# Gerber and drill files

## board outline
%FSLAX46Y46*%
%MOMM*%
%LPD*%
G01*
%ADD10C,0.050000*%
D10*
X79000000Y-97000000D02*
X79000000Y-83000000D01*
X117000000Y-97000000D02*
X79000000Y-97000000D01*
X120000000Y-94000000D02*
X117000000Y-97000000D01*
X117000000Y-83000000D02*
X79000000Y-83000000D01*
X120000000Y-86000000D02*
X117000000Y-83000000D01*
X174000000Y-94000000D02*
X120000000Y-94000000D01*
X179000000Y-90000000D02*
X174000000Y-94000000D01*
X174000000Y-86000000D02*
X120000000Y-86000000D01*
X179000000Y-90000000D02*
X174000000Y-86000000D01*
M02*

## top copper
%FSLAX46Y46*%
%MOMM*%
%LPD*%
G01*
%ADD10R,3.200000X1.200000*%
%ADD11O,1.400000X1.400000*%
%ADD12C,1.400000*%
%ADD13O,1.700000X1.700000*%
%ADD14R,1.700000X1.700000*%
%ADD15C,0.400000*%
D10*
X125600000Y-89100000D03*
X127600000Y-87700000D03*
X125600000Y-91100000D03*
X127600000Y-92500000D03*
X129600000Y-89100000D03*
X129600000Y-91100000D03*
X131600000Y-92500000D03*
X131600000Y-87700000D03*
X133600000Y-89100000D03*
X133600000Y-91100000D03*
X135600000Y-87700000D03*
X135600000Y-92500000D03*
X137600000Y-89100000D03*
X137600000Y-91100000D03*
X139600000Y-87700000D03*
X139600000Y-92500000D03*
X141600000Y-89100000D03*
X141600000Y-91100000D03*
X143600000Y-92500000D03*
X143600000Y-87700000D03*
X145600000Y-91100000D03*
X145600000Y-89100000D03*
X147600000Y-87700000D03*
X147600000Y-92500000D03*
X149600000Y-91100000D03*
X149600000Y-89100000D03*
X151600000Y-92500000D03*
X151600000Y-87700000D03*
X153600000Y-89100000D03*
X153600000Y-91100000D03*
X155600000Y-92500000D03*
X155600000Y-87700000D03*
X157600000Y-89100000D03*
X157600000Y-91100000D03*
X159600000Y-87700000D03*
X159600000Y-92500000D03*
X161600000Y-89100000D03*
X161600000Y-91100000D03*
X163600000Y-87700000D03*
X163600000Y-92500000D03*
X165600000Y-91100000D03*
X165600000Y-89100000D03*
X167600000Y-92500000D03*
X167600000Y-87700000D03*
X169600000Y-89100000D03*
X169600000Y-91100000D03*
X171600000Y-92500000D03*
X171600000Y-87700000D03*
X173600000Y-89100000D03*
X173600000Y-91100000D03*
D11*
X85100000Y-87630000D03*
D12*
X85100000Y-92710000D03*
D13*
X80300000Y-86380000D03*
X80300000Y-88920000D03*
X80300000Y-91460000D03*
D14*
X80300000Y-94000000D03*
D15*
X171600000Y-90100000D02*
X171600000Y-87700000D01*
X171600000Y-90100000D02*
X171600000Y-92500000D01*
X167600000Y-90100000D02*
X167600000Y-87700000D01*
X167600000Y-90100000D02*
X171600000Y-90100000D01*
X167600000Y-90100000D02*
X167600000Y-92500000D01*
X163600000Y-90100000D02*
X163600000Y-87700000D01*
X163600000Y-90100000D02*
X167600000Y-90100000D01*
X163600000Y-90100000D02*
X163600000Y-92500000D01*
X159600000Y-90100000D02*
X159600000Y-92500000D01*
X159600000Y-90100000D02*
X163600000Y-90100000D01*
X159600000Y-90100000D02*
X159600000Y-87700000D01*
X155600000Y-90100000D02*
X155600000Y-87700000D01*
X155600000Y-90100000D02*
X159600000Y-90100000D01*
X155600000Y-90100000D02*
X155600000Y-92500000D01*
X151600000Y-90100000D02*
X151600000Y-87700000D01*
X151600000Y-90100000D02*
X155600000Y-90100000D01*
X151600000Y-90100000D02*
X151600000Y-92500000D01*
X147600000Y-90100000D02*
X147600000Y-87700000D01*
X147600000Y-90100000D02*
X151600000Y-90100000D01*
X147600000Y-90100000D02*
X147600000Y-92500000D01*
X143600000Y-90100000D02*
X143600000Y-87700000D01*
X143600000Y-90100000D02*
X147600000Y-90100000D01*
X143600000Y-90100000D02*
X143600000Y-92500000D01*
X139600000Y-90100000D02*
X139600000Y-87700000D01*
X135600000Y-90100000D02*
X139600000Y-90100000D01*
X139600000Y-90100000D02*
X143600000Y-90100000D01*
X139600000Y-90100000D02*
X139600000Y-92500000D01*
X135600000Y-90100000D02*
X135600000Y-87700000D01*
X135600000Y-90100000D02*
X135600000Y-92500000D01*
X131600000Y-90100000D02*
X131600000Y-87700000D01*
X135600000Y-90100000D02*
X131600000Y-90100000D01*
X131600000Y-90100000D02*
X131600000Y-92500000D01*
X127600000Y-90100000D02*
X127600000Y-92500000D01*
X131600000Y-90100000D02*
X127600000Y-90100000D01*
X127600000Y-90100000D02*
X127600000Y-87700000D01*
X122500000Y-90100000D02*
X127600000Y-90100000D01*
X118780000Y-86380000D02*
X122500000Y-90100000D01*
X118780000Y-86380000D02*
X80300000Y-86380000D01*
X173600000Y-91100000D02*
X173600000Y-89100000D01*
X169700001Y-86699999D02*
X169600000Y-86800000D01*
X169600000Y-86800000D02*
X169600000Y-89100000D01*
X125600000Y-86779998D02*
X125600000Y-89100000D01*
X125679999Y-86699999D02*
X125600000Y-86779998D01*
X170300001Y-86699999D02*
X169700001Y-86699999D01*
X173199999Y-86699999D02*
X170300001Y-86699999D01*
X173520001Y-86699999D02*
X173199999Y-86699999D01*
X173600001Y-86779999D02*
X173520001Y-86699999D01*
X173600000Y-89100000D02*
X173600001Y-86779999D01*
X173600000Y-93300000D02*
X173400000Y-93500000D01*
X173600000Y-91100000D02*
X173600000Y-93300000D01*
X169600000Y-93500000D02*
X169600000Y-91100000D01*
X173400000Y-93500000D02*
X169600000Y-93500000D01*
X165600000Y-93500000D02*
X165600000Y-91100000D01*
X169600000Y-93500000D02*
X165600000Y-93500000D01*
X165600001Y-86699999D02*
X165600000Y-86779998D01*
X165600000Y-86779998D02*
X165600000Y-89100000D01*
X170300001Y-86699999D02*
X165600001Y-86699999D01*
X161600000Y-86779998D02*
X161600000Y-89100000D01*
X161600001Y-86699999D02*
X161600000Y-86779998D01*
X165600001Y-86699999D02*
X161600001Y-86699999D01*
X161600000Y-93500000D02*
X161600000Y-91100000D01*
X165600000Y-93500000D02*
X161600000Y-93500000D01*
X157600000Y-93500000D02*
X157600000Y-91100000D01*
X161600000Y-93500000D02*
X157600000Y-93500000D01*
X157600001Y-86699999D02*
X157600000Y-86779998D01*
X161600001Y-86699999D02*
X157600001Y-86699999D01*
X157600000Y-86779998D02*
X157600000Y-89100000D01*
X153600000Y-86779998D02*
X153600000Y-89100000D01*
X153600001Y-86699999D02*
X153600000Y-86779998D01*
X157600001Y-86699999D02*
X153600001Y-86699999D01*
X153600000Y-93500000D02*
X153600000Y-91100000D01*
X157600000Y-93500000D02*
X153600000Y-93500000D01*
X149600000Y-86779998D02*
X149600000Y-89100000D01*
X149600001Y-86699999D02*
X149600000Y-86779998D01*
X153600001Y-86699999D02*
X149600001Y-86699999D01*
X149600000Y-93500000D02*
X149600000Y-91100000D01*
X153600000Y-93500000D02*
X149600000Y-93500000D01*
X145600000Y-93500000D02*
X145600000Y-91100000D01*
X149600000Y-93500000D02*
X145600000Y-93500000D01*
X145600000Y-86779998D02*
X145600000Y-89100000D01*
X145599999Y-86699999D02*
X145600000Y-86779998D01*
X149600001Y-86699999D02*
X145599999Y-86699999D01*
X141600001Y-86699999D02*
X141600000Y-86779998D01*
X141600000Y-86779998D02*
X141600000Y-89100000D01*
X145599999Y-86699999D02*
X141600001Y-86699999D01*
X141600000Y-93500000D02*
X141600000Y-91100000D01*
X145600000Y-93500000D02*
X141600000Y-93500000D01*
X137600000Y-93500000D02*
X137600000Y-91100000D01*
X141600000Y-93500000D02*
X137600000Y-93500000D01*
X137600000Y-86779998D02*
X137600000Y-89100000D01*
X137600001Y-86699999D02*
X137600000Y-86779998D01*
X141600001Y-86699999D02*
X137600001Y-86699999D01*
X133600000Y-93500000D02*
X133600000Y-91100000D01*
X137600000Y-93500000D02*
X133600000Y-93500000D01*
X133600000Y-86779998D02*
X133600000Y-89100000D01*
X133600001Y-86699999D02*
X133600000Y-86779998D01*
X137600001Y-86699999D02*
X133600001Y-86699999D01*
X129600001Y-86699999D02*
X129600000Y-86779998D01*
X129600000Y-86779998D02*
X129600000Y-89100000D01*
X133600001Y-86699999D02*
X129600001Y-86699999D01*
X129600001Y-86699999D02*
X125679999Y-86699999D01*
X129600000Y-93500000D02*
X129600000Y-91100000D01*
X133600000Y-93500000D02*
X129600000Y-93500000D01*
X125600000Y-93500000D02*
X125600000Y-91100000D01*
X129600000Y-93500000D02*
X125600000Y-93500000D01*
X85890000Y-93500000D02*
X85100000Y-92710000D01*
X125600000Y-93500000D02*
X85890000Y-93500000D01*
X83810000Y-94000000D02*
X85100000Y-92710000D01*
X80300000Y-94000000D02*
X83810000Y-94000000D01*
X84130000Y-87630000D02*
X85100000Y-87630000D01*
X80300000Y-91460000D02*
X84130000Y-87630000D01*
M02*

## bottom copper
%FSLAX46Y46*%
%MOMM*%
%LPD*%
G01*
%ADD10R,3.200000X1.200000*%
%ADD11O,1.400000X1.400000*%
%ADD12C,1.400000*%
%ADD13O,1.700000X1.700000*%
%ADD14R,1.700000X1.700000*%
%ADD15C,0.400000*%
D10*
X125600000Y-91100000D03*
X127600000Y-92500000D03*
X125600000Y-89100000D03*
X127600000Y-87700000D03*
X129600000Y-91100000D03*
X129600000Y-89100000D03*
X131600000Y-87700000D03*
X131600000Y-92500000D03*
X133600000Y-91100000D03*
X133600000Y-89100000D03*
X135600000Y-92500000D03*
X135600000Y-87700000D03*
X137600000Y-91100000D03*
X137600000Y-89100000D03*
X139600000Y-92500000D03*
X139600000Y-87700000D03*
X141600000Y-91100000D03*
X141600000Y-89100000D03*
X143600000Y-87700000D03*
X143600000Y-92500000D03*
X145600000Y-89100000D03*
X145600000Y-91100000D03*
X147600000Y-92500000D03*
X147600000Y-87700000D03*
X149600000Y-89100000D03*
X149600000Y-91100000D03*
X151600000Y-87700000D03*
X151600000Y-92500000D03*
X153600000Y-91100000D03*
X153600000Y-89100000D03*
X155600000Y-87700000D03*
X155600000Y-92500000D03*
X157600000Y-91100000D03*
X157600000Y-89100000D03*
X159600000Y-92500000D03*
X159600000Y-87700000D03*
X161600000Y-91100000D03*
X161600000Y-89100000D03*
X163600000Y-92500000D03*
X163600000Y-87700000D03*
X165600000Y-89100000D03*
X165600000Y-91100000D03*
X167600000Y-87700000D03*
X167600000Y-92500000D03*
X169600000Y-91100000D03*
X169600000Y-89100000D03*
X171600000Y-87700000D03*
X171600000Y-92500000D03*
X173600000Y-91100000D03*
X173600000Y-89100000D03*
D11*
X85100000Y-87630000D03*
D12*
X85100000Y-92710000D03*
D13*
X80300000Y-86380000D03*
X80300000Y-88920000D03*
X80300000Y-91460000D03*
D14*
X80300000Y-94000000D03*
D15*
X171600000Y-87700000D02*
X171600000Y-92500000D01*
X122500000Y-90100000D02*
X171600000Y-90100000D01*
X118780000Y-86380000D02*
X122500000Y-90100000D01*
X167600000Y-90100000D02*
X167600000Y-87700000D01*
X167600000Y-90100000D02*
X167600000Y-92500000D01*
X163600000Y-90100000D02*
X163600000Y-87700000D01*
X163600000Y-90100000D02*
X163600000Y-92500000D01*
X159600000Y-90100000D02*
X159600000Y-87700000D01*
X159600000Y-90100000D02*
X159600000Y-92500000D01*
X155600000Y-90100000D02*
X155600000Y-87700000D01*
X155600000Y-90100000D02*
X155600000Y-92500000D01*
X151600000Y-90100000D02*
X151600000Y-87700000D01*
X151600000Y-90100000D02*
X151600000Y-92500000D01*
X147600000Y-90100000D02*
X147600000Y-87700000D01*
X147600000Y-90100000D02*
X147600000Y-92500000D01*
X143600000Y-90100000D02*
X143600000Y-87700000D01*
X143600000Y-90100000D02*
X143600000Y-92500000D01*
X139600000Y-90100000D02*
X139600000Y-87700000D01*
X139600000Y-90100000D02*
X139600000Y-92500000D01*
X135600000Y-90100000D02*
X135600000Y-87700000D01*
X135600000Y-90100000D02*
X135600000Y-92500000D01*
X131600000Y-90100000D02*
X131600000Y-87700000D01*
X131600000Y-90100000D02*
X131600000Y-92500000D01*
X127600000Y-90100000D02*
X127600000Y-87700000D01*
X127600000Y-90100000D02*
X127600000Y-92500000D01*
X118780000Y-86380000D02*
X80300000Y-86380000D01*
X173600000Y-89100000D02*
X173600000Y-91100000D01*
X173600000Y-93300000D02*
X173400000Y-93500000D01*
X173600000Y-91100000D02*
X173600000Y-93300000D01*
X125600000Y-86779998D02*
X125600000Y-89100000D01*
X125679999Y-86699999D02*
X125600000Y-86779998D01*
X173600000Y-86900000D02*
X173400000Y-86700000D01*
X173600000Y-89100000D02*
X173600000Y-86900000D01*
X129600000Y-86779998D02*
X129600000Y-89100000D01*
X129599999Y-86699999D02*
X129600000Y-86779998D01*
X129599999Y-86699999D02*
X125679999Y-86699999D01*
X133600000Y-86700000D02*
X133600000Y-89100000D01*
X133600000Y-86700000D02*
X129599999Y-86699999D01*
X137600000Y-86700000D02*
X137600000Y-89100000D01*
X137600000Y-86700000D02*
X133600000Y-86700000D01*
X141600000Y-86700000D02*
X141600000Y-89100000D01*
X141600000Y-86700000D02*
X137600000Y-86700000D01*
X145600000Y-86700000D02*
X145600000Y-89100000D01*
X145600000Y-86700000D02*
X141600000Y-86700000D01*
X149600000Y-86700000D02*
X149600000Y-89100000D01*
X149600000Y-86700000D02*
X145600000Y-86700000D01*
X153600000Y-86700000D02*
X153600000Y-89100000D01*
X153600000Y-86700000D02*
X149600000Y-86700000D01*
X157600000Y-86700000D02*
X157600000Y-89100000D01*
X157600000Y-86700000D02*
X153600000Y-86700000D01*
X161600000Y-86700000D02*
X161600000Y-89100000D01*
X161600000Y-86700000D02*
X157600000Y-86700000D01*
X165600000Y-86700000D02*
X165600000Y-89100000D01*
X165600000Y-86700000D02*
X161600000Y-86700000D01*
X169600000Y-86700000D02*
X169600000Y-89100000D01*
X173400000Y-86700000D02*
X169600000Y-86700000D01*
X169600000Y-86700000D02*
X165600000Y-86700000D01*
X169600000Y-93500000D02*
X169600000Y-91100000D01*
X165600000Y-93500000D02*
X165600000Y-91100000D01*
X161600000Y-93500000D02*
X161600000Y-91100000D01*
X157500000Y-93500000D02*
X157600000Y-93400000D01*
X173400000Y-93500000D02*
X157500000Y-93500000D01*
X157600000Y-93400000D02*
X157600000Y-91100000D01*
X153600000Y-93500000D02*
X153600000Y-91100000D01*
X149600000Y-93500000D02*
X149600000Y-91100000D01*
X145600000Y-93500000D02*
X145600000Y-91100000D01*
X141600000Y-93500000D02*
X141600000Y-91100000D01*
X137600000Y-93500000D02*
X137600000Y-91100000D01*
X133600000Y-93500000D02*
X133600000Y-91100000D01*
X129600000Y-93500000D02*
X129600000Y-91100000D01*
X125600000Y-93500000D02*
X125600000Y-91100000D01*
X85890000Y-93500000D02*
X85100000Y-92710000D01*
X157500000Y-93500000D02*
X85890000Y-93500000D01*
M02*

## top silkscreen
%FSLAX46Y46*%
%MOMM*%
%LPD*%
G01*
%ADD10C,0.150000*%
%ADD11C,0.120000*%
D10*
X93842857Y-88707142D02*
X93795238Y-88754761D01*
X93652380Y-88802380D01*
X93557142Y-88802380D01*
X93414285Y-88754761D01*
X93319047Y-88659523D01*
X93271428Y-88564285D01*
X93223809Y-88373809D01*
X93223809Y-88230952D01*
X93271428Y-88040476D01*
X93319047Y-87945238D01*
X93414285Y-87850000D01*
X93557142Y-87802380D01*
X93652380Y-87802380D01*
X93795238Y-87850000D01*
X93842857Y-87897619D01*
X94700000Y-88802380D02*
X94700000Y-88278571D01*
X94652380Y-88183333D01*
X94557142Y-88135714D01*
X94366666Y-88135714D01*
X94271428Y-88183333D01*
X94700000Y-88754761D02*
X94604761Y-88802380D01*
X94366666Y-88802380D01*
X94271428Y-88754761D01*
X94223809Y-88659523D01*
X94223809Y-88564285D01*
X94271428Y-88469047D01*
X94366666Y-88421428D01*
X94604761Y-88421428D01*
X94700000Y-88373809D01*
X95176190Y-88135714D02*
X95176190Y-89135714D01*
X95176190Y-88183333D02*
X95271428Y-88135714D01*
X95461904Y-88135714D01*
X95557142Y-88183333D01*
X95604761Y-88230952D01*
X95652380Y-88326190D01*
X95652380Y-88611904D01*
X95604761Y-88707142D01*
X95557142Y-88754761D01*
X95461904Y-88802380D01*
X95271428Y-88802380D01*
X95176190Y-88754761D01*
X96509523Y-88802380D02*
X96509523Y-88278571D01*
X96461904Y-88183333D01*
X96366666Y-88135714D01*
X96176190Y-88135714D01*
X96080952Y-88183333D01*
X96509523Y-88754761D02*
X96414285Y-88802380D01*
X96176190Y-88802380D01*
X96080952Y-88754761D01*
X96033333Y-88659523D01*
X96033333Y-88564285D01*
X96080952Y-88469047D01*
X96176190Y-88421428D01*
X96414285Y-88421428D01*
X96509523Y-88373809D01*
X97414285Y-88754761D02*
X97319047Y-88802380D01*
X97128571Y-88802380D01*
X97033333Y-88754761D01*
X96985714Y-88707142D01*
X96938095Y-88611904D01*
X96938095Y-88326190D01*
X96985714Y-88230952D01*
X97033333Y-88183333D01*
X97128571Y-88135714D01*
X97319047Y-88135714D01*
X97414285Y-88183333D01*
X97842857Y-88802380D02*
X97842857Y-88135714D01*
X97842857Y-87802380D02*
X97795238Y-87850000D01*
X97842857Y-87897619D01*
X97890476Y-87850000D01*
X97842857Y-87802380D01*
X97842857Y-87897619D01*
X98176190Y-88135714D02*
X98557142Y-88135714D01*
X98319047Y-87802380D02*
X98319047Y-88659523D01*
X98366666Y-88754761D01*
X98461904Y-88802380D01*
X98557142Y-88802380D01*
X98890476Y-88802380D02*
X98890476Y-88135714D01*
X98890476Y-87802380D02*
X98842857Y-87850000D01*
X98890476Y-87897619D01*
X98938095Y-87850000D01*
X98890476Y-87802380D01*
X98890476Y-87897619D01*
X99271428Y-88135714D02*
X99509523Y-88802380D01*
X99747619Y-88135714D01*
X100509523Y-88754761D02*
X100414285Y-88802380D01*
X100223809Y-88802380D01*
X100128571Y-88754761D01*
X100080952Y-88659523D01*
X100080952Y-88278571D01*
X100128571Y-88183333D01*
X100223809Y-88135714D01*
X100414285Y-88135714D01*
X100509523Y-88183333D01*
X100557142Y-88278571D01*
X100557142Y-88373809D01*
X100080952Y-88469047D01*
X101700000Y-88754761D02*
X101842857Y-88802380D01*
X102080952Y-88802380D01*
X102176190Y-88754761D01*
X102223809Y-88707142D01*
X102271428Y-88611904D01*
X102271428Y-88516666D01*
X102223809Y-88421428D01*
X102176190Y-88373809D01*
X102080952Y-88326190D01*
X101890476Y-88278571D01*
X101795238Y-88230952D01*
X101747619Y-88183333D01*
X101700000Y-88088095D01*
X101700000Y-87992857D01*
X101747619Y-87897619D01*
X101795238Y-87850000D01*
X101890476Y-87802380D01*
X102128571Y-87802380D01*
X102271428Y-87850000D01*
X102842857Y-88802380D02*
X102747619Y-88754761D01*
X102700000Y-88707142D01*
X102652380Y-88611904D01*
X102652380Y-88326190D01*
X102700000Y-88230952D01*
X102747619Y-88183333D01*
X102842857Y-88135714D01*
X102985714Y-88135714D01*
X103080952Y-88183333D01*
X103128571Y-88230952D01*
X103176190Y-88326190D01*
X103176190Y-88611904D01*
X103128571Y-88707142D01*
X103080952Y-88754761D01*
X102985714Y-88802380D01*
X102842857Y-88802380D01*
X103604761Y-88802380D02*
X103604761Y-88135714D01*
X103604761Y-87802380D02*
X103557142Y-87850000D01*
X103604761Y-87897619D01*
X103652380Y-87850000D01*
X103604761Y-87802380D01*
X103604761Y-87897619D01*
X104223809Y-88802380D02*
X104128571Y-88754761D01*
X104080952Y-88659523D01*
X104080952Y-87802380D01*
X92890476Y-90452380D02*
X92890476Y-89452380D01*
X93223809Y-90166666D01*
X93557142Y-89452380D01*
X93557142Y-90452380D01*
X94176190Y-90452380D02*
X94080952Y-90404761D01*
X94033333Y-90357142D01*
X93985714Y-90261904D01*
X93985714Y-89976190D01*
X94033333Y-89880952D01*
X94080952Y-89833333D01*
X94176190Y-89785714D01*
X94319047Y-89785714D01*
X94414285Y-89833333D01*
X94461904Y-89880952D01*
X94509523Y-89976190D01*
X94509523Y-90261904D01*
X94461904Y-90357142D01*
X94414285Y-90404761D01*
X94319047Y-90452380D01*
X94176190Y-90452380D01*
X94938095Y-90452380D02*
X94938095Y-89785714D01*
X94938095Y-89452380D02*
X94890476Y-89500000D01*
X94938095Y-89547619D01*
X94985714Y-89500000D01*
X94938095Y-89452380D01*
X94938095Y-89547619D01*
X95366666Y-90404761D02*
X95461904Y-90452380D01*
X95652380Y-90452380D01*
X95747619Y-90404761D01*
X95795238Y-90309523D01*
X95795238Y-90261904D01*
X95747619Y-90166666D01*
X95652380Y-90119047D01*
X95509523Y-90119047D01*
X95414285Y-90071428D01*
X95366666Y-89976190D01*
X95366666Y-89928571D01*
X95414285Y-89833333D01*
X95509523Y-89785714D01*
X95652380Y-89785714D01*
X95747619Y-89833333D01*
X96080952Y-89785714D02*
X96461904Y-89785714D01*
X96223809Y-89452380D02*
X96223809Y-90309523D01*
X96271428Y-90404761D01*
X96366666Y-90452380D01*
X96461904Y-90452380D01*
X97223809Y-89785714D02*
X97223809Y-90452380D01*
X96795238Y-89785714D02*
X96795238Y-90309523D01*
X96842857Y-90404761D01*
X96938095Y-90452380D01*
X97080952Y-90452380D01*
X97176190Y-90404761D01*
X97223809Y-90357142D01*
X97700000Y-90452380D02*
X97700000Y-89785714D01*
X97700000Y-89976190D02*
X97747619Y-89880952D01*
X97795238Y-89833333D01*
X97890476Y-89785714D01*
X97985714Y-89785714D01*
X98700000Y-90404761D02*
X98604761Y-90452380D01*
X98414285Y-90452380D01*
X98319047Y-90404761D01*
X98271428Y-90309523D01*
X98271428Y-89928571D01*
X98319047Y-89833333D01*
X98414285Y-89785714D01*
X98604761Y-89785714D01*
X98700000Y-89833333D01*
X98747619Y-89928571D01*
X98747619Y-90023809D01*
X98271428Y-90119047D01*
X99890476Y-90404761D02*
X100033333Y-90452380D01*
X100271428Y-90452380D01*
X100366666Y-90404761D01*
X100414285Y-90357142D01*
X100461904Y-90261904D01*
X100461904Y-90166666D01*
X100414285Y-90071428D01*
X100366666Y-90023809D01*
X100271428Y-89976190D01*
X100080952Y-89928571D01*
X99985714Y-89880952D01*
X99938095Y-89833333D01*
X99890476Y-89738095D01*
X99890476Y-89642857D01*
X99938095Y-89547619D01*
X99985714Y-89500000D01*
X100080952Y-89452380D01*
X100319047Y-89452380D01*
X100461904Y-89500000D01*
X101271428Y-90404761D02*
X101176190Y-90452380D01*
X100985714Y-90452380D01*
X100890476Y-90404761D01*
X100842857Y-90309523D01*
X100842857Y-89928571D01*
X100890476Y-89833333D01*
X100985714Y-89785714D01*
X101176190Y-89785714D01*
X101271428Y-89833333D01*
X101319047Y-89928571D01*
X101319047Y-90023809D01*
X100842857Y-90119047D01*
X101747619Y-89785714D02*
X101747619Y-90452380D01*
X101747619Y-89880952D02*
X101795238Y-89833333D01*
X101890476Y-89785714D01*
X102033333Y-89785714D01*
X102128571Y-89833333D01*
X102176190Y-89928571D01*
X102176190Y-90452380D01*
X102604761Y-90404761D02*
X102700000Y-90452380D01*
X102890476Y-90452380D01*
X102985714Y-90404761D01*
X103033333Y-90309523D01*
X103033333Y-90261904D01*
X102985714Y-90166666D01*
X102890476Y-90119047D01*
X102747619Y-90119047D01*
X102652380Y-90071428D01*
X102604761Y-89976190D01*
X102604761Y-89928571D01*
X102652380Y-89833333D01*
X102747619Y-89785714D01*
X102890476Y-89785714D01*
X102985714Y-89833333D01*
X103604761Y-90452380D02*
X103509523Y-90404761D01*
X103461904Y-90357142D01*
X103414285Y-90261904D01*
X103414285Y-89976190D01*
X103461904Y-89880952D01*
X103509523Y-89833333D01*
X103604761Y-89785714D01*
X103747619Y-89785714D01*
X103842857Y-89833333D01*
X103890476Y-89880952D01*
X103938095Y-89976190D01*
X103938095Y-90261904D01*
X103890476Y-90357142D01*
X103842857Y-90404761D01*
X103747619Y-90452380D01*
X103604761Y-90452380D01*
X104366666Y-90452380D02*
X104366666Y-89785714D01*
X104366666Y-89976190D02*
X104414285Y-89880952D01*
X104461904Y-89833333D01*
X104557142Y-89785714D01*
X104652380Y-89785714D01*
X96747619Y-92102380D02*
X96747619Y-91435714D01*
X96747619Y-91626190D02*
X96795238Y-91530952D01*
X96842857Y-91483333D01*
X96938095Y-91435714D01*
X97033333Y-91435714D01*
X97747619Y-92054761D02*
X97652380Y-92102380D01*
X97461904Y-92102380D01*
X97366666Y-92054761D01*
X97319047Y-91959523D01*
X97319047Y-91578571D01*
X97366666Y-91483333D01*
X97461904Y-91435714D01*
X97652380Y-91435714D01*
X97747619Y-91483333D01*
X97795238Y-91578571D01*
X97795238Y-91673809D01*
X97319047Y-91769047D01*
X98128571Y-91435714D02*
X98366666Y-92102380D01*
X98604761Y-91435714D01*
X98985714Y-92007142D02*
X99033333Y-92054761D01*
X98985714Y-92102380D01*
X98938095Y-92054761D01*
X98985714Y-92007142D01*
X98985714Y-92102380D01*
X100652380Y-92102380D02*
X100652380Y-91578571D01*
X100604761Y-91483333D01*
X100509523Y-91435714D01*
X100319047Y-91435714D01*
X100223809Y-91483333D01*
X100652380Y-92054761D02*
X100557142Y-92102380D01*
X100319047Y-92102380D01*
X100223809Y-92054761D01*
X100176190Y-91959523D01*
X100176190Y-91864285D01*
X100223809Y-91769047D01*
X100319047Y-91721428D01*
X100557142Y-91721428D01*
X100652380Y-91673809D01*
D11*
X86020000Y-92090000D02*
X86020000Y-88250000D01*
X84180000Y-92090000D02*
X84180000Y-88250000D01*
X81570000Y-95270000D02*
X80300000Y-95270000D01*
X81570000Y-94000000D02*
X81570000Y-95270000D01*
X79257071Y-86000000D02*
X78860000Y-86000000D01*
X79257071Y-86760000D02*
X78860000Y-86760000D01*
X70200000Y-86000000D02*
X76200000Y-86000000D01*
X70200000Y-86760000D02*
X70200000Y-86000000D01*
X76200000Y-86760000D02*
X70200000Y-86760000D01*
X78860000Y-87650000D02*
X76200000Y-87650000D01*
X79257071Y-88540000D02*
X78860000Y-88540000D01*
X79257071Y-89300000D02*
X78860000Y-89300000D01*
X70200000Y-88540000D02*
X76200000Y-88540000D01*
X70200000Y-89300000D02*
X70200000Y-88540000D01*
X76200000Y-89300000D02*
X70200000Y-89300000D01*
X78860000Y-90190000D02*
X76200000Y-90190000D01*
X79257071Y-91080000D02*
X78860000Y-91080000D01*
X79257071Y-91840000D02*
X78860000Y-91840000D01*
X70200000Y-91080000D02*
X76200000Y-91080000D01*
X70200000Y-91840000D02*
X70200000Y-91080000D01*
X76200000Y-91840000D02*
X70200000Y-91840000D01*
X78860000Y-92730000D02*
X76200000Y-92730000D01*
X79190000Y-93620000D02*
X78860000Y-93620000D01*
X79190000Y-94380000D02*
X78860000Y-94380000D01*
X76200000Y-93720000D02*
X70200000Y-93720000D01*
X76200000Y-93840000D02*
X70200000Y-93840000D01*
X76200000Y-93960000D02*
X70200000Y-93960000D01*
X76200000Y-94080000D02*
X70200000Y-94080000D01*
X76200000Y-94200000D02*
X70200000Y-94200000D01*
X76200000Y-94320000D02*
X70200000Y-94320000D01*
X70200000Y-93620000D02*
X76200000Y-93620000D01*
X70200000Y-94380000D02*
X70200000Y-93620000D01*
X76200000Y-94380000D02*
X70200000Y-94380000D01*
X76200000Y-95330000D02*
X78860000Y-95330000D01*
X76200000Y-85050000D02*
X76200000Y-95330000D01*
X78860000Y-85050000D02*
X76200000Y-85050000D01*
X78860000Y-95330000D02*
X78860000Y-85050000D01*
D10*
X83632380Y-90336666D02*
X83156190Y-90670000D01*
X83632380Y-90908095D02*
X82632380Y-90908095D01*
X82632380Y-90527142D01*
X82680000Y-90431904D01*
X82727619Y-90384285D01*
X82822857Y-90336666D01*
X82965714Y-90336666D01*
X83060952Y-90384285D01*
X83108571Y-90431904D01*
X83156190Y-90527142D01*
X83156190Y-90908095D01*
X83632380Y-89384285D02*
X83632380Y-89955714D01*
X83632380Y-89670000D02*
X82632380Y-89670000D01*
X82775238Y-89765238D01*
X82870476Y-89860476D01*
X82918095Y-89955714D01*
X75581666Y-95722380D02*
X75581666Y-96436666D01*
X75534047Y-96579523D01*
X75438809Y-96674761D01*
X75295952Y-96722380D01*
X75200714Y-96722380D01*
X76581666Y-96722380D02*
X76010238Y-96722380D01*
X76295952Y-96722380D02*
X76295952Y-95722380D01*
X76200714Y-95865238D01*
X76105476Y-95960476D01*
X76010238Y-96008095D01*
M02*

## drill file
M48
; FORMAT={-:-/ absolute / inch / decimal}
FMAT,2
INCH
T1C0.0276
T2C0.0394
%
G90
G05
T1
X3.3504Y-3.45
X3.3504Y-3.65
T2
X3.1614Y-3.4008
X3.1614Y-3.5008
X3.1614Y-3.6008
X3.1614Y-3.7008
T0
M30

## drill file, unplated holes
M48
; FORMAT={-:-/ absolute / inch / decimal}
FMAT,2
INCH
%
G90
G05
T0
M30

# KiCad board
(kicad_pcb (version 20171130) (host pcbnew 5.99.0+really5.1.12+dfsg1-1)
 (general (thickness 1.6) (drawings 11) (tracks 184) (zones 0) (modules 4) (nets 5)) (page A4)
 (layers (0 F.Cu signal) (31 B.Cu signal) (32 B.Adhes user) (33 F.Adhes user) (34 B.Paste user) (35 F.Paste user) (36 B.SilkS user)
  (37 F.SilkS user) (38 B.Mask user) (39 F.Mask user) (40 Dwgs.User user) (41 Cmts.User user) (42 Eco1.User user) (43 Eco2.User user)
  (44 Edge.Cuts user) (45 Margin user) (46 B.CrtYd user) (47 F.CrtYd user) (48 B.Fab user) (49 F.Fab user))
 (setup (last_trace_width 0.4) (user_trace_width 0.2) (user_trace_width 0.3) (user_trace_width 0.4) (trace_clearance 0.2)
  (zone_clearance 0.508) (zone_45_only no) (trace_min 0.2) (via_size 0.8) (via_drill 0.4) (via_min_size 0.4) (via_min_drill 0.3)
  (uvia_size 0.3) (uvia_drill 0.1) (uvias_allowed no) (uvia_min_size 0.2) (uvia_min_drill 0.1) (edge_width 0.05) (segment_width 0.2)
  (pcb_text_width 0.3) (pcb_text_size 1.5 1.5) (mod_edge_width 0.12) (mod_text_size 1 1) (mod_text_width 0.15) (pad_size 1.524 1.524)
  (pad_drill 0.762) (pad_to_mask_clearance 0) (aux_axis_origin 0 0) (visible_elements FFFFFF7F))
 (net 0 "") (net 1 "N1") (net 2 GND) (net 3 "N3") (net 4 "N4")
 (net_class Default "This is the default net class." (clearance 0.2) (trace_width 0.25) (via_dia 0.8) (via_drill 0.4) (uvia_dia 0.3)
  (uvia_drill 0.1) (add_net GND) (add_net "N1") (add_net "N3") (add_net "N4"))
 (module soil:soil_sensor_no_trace (layer B.Cu) (at 124 90.1)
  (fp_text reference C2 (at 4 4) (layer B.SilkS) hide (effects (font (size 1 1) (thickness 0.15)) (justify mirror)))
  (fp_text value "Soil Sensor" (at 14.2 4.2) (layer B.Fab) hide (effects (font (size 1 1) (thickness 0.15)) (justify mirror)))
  (pad 1 smd rect (at 1.6 1) (size 3.2 1.2) (layers B.Cu) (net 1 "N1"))
  (pad 2 smd rect (at 3.6 2.4) (size 3.2 1.2) (layers B.Cu) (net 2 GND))
  (pad 1 smd rect (at 1.6 -1) (size 3.2 1.2) (layers B.Cu) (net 1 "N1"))
  (pad 2 smd rect (at 3.6 -2.4) (size 3.2 1.2) (layers B.Cu) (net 2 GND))
  (pad 1 smd rect (at 5.6 1) (size 3.2 1.2) (layers B.Cu) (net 1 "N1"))
  (pad 1 smd rect (at 5.6 -1) (size 3.2 1.2) (layers B.Cu) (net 1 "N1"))
  (pad 2 smd rect (at 7.6 -2.4) (size 3.2 1.2) (layers B.Cu) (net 2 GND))
  (pad 2 smd rect (at 7.6 2.4) (size 3.2 1.2) (layers B.Cu) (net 2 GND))
  (pad 1 smd rect (at 9.6 1) (size 3.2 1.2) (layers B.Cu) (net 1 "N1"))
  (pad 1 smd rect (at 9.6 -1) (size 3.2 1.2) (layers B.Cu) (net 1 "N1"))
  (pad 2 smd rect (at 11.6 2.4) (size 3.2 1.2) (layers B.Cu) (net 2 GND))
  (pad 2 smd rect (at 11.6 -2.4) (size 3.2 1.2) (layers B.Cu) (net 2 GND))
  (pad 1 smd rect (at 13.6 1) (size 3.2 1.2) (layers B.Cu) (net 1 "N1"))
  (pad 1 smd rect (at 13.6 -1) (size 3.2 1.2) (layers B.Cu) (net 1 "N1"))
  (pad 2 smd rect (at 15.6 2.4) (size 3.2 1.2) (layers B.Cu) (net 2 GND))
  (pad 2 smd rect (at 15.6 -2.4) (size 3.2 1.2) (layers B.Cu) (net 2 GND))
  (pad 1 smd rect (at 17.6 1) (size 3.2 1.2) (layers B.Cu) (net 1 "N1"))
  (pad 1 smd rect (at 17.6 -1) (size 3.2 1.2) (layers B.Cu) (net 1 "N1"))
  (pad 2 smd rect (at 19.6 -2.4) (size 3.2 1.2) (layers B.Cu) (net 2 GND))
  (pad 2 smd rect (at 19.6 2.4) (size 3.2 1.2) (layers B.Cu) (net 2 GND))
  (pad 1 smd rect (at 21.6 -1) (size 3.2 1.2) (layers B.Cu) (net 1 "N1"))
  (pad 1 smd rect (at 21.6 1) (size 3.2 1.2) (layers B.Cu) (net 1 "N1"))
  (pad 2 smd rect (at 23.6 2.4) (size 3.2 1.2) (layers B.Cu) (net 2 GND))
  (pad 2 smd rect (at 23.6 -2.4) (size 3.2 1.2) (layers B.Cu) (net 2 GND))
  (pad 1 smd rect (at 25.6 -1) (size 3.2 1.2) (layers B.Cu) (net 1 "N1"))
  (pad 1 smd rect (at 25.6 1) (size 3.2 1.2) (layers B.Cu) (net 1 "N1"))
  (pad 2 smd rect (at 27.6 -2.4) (size 3.2 1.2) (layers B.Cu) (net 2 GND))
  (pad 2 smd rect (at 27.6 2.4) (size 3.2 1.2) (layers B.Cu) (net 2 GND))
  (pad 1 smd rect (at 29.6 1) (size 3.2 1.2) (layers B.Cu) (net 1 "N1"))
  (pad 1 smd rect (at 29.6 -1) (size 3.2 1.2) (layers B.Cu) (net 1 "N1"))
  (pad 2 smd rect (at 31.6 -2.4) (size 3.2 1.2) (layers B.Cu) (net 2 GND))
  (pad 2 smd rect (at 31.6 2.4) (size 3.2 1.2) (layers B.Cu) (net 2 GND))
  (pad 1 smd rect (at 33.6 1) (size 3.2 1.2) (layers B.Cu) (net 1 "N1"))
  (pad 1 smd rect (at 33.6 -1) (size 3.2 1.2) (layers B.Cu) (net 1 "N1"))
  (pad 2 smd rect (at 35.6 2.4) (size 3.2 1.2) (layers B.Cu) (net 2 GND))
  (pad 2 smd rect (at 35.6 -2.4) (size 3.2 1.2) (layers B.Cu) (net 2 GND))
  (pad 1 smd rect (at 37.6 1) (size 3.2 1.2) (layers B.Cu) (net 1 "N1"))
  (pad 1 smd rect (at 37.6 -1) (size 3.2 1.2) (layers B.Cu) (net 1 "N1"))
  (pad 2 smd rect (at 39.6 2.4) (size 3.2 1.2) (layers B.Cu) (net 2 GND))
  (pad 2 smd rect (at 39.6 -2.4) (size 3.2 1.2) (layers B.Cu) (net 2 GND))
  (pad 1 smd rect (at 41.6 -1) (size 3.2 1.2) (layers B.Cu) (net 1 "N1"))
  (pad 1 smd rect (at 41.6 1) (size 3.2 1.2) (layers B.Cu) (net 1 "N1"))
  (pad 2 smd rect (at 43.6 -2.4) (size 3.2 1.2) (layers B.Cu) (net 2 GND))
  (pad 2 smd rect (at 43.6 2.4) (size 3.2 1.2) (layers B.Cu) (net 2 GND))
  (pad 1 smd rect (at 45.6 1) (size 3.2 1.2) (layers B.Cu) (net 1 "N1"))
  (pad 1 smd rect (at 45.6 -1) (size 3.2 1.2) (layers B.Cu) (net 1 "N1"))
  (pad 2 smd rect (at 47.6 -2.4) (size 3.2 1.2) (layers B.Cu) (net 2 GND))
  (pad 2 smd rect (at 47.6 2.4) (size 3.2 1.2) (layers B.Cu) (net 2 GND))
  (pad 1 smd rect (at 49.6 1) (size 3.2 1.2) (layers B.Cu) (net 1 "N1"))
  (pad 1 smd rect (at 49.6 -1) (size 3.2 1.2) (layers B.Cu) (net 1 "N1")))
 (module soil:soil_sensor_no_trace (layer F.Cu) (at 124 90.1)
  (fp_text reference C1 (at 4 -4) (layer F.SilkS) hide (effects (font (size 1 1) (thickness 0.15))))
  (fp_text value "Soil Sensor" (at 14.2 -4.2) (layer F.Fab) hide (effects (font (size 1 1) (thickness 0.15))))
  (pad 1 smd rect (at 1.6 -1) (size 3.2 1.2) (layers F.Cu) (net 1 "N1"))
  (pad 2 smd rect (at 3.6 -2.4) (size 3.2 1.2) (layers F.Cu) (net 2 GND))
  (pad 1 smd rect (at 1.6 1) (size 3.2 1.2) (layers F.Cu) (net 1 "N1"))
  (pad 2 smd rect (at 3.6 2.4) (size 3.2 1.2) (layers F.Cu) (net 2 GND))
  (pad 1 smd rect (at 5.6 -1) (size 3.2 1.2) (layers F.Cu) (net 1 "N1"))
  (pad 1 smd rect (at 5.6 1) (size 3.2 1.2) (layers F.Cu) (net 1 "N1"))
  (pad 2 smd rect (at 7.6 2.4) (size 3.2 1.2) (layers F.Cu) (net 2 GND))
  (pad 2 smd rect (at 7.6 -2.4) (size 3.2 1.2) (layers F.Cu) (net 2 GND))
  (pad 1 smd rect (at 9.6 -1) (size 3.2 1.2) (layers F.Cu) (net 1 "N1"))
  (pad 1 smd rect (at 9.6 1) (size 3.2 1.2) (layers F.Cu) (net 1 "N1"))
  (pad 2 smd rect (at 11.6 -2.4) (size 3.2 1.2) (layers F.Cu) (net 2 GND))
  (pad 2 smd rect (at 11.6 2.4) (size 3.2 1.2) (layers F.Cu) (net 2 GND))
  (pad 1 smd rect (at 13.6 -1) (size 3.2 1.2) (layers F.Cu) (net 1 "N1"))
  (pad 1 smd rect (at 13.6 1) (size 3.2 1.2) (layers F.Cu) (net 1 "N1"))
  (pad 2 smd rect (at 15.6 -2.4) (size 3.2 1.2) (layers F.Cu) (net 2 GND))
  (pad 2 smd rect (at 15.6 2.4) (size 3.2 1.2) (layers F.Cu) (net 2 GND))
  (pad 1 smd rect (at 17.6 -1) (size 3.2 1.2) (layers F.Cu) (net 1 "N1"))
  (pad 1 smd rect (at 17.6 1) (size 3.2 1.2) (layers F.Cu) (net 1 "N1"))
  (pad 2 smd rect (at 19.6 2.4) (size 3.2 1.2) (layers F.Cu) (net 2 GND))
  (pad 2 smd rect (at 19.6 -2.4) (size 3.2 1.2) (layers F.Cu) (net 2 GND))
  (pad 1 smd rect (at 21.6 1) (size 3.2 1.2) (layers F.Cu) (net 1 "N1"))
  (pad 1 smd rect (at 21.6 -1) (size 3.2 1.2) (layers F.Cu) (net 1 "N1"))
  (pad 2 smd rect (at 23.6 -2.4) (size 3.2 1.2) (layers F.Cu) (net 2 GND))
  (pad 2 smd rect (at 23.6 2.4) (size 3.2 1.2) (layers F.Cu) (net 2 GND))
  (pad 1 smd rect (at 25.6 1) (size 3.2 1.2) (layers F.Cu) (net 1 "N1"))
  (pad 1 smd rect (at 25.6 -1) (size 3.2 1.2) (layers F.Cu) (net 1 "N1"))
  (pad 2 smd rect (at 27.6 2.4) (size 3.2 1.2) (layers F.Cu) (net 2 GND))
  (pad 2 smd rect (at 27.6 -2.4) (size 3.2 1.2) (layers F.Cu) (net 2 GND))
  (pad 1 smd rect (at 29.6 -1) (size 3.2 1.2) (layers F.Cu) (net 1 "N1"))
  (pad 1 smd rect (at 29.6 1) (size 3.2 1.2) (layers F.Cu) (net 1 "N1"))
  (pad 2 smd rect (at 31.6 2.4) (size 3.2 1.2) (layers F.Cu) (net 2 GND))
  (pad 2 smd rect (at 31.6 -2.4) (size 3.2 1.2) (layers F.Cu) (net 2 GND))
  (pad 1 smd rect (at 33.6 -1) (size 3.2 1.2) (layers F.Cu) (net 1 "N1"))
  (pad 1 smd rect (at 33.6 1) (size 3.2 1.2) (layers F.Cu) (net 1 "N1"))
  (pad 2 smd rect (at 35.6 -2.4) (size 3.2 1.2) (layers F.Cu) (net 2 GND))
  (pad 2 smd rect (at 35.6 2.4) (size 3.2 1.2) (layers F.Cu) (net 2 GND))
  (pad 1 smd rect (at 37.6 -1) (size 3.2 1.2) (layers F.Cu) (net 1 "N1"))
  (pad 1 smd rect (at 37.6 1) (size 3.2 1.2) (layers F.Cu) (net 1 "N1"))
  (pad 2 smd rect (at 39.6 -2.4) (size 3.2 1.2) (layers F.Cu) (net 2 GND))
  (pad 2 smd rect (at 39.6 2.4) (size 3.2 1.2) (layers F.Cu) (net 2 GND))
  (pad 1 smd rect (at 41.6 1) (size 3.2 1.2) (layers F.Cu) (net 1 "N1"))
  (pad 1 smd rect (at 41.6 -1) (size 3.2 1.2) (layers F.Cu) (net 1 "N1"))
  (pad 2 smd rect (at 43.6 2.4) (size 3.2 1.2) (layers F.Cu) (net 2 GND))
  (pad 2 smd rect (at 43.6 -2.4) (size 3.2 1.2) (layers F.Cu) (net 2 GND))
  (pad 1 smd rect (at 45.6 -1) (size 3.2 1.2) (layers F.Cu) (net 1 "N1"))
  (pad 1 smd rect (at 45.6 1) (size 3.2 1.2) (layers F.Cu) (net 1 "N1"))
  (pad 2 smd rect (at 47.6 2.4) (size 3.2 1.2) (layers F.Cu) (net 2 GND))
  (pad 2 smd rect (at 47.6 -2.4) (size 3.2 1.2) (layers F.Cu) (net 2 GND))
  (pad 1 smd rect (at 49.6 -1) (size 3.2 1.2) (layers F.Cu) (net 1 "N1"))
  (pad 1 smd rect (at 49.6 1) (size 3.2 1.2) (layers F.Cu) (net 1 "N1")))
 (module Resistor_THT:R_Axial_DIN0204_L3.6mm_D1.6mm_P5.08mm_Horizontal (layer F.Cu) (at 85.1 92.71 90)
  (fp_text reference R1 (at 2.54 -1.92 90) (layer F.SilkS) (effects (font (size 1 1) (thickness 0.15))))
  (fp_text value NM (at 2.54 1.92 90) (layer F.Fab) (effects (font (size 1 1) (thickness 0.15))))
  (fp_line (start 0.62 -0.92) (end 4.46 -0.92) (layer F.SilkS) (width 0.12))
  (fp_line (start 0.62 0.92) (end 4.46 0.92) (layer F.SilkS) (width 0.12))
  (pad 2 thru_hole oval (at 5.08 0 90) (size 1.4 1.4) (drill 0.7) (layers *.Cu *.Mask) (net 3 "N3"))
  (pad 1 thru_hole circle (at 0 0 90) (size 1.4 1.4) (drill 0.7) (layers *.Cu *.Mask) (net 1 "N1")))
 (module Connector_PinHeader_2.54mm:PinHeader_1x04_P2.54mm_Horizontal (layer F.Cu) (at 80.3 94 180)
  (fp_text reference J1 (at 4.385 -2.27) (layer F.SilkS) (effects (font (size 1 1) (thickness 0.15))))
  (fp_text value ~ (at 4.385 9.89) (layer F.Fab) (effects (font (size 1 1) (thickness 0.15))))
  (fp_line (start 1.44 -1.33) (end 1.44 8.95) (layer F.SilkS) (width 0.12))
  (fp_line (start 1.44 8.95) (end 4.1 8.95) (layer F.SilkS) (width 0.12))
  (fp_line (start 4.1 8.95) (end 4.1 -1.33) (layer F.SilkS) (width 0.12))
  (fp_line (start 4.1 -1.33) (end 1.44 -1.33) (layer F.SilkS) (width 0.12))
  (fp_line (start 4.1 -0.38) (end 10.1 -0.38) (layer F.SilkS) (width 0.12))
  (fp_line (start 10.1 -0.38) (end 10.1 0.38) (layer F.SilkS) (width 0.12))
  (fp_line (start 10.1 0.38) (end 4.1 0.38) (layer F.SilkS) (width 0.12))
  (fp_line (start 4.1 -0.32) (end 10.1 -0.32) (layer F.SilkS) (width 0.12))
  (fp_line (start 4.1 -0.2) (end 10.1 -0.2) (layer F.SilkS) (width 0.12))
  (fp_line (start 4.1 -0.08) (end 10.1 -0.08) (layer F.SilkS) (width 0.12))
  (fp_line (start 4.1 0.04) (end 10.1 0.04) (layer F.SilkS) (width 0.12))
  (fp_line (start 4.1 0.16) (end 10.1 0.16) (layer F.SilkS) (width 0.12))
  (fp_line (start 4.1 0.28) (end 10.1 0.28) (layer F.SilkS) (width 0.12))
  (fp_line (start 1.11 -0.38) (end 1.44 -0.38) (layer F.SilkS) (width 0.12))
  (fp_line (start 1.11 0.38) (end 1.44 0.38) (layer F.SilkS) (width 0.12))
  (fp_line (start 1.44 1.27) (end 4.1 1.27) (layer F.SilkS) (width 0.12))
  (fp_line (start 4.1 2.16) (end 10.1 2.16) (layer F.SilkS) (width 0.12))
  (fp_line (start 10.1 2.16) (end 10.1 2.92) (layer F.SilkS) (width 0.12))
  (fp_line (start 10.1 2.92) (end 4.1 2.92) (layer F.SilkS) (width 0.12))
  (fp_line (start 1.042929 2.16) (end 1.44 2.16) (layer F.SilkS) (width 0.12))
  (fp_line (start 1.042929 2.92) (end 1.44 2.92) (layer F.SilkS) (width 0.12))
  (fp_line (start 1.44 3.81) (end 4.1 3.81) (layer F.SilkS) (width 0.12))
  (fp_line (start 4.1 4.7) (end 10.1 4.7) (layer F.SilkS) (width 0.12))
  (fp_line (start 10.1 4.7) (end 10.1 5.46) (layer F.SilkS) (width 0.12))
  (fp_line (start 10.1 5.46) (end 4.1 5.46) (layer F.SilkS) (width 0.12))
  (fp_line (start 1.042929 4.7) (end 1.44 4.7) (layer F.SilkS) (width 0.12))
  (fp_line (start 1.042929 5.46) (end 1.44 5.46) (layer F.SilkS) (width 0.12))
  (fp_line (start 1.44 6.35) (end 4.1 6.35) (layer F.SilkS) (width 0.12))
  (fp_line (start 4.1 7.24) (end 10.1 7.24) (layer F.SilkS) (width 0.12))
  (fp_line (start 10.1 7.24) (end 10.1 8) (layer F.SilkS) (width 0.12))
  (fp_line (start 10.1 8) (end 4.1 8) (layer F.SilkS) (width 0.12))
  (fp_line (start 1.042929 7.24) (end 1.44 7.24) (layer F.SilkS) (width 0.12))
  (fp_line (start 1.042929 8) (end 1.44 8) (layer F.SilkS) (width 0.12))
  (fp_line (start -1.27 0) (end -1.27 -1.27) (layer F.SilkS) (width 0.12))
  (fp_line (start -1.27 -1.27) (end 0 -1.27) (layer F.SilkS) (width 0.12))
  (pad 4 thru_hole oval (at 0 7.62 180) (size 1.7 1.7) (drill 1) (layers *.Cu *.Mask) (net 2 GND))
  (pad 3 thru_hole oval (at 0 5.08 180) (size 1.7 1.7) (drill 1) (layers *.Cu *.Mask) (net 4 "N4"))
  (pad 2 thru_hole oval (at 0 2.54 180) (size 1.7 1.7) (drill 1) (layers *.Cu *.Mask) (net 3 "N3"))
  (pad 1 thru_hole rect (at 0 0 180) (size 1.7 1.7) (drill 1) (layers *.Cu *.Mask) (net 1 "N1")))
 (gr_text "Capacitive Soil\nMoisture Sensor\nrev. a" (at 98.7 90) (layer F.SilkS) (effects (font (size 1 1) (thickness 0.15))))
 (gr_line (start 79 97) (end 79 83) (layer Edge.Cuts) (width 0.05))
 (gr_line (start 117 97) (end 79 97) (layer Edge.Cuts) (width 0.05))
 (gr_line (start 120 94) (end 117 97) (layer Edge.Cuts) (width 0.05))
 (gr_line (start 117 83) (end 79 83) (layer Edge.Cuts) (width 0.05))
 (gr_line (start 120 86) (end 117 83) (layer Edge.Cuts) (width 0.05))
 (gr_line (start 174 94) (end 120 94) (layer Edge.Cuts) (width 0.05))
 (gr_line (start 179 90) (end 174 94) (layer Edge.Cuts) (width 0.05))
 (gr_line (start 174 86) (end 120 86) (layer Edge.Cuts) (width 0.05))
 (gr_line (start 179 90) (end 174 86) (layer Edge.Cuts) (width 0.05))
 (segment (start 171.6 90.1) (end 171.6 87.7) (width 0.4) (layer F.Cu) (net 2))
 (segment (start 171.6 90.1) (end 171.6 92.5) (width 0.4) (layer F.Cu) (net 2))
 (segment (start 167.6 90.1) (end 167.6 87.7) (width 0.4) (layer F.Cu) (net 2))
 (segment (start 167.6 90.1) (end 171.6 90.1) (width 0.4) (layer F.Cu) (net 2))
 (segment (start 167.6 90.1) (end 167.6 92.5) (width 0.4) (layer F.Cu) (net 2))
 (segment (start 163.6 90.1) (end 163.6 87.7) (width 0.4) (layer F.Cu) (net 2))
 (segment (start 163.6 90.1) (end 167.6 90.1) (width 0.4) (layer F.Cu) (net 2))
 (segment (start 163.6 90.1) (end 163.6 92.5) (width 0.4) (layer F.Cu) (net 2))
 (segment (start 159.6 90.1) (end 159.6 92.5) (width 0.4) (layer F.Cu) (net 2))
 (segment (start 159.6 90.1) (end 163.6 90.1) (width 0.4) (layer F.Cu) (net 2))
 (segment (start 159.6 90.1) (end 159.6 87.7) (width 0.4) (layer F.Cu) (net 2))
 (segment (start 155.6 90.1) (end 155.6 87.7) (width 0.4) (layer F.Cu) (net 2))
 (segment (start 155.6 90.1) (end 159.6 90.1) (width 0.4) (layer F.Cu) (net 2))
 (segment (start 155.6 90.1) (end 155.6 92.5) (width 0.4) (layer F.Cu) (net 2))
 (segment (start 151.6 90.1) (end 151.6 87.7) (width 0.4) (layer F.Cu) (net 2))
 (segment (start 151.6 90.1) (end 155.6 90.1) (width 0.4) (layer F.Cu) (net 2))
 (segment (start 151.6 90.1) (end 151.6 92.5) (width 0.4) (layer F.Cu) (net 2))
 (segment (start 147.6 90.1) (end 147.6 87.7) (width 0.4) (layer F.Cu) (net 2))
 (segment (start 147.6 90.1) (end 151.6 90.1) (width 0.4) (layer F.Cu) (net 2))
 (segment (start 147.6 90.1) (end 147.6 92.5) (width 0.4) (layer F.Cu) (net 2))
 (segment (start 143.6 90.1) (end 143.6 87.7) (width 0.4) (layer F.Cu) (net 2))
 (segment (start 143.6 90.1) (end 147.6 90.1) (width 0.4) (layer F.Cu) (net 2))
 (segment (start 143.6 90.1) (end 143.6 92.5) (width 0.4) (layer F.Cu) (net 2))
 (segment (start 139.6 90.1) (end 139.6 87.7) (width 0.4) (layer F.Cu) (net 2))
 (segment (start 135.6 90.1) (end 139.6 90.1) (width 0.4) (layer F.Cu) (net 2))
 (segment (start 139.6 90.1) (end 143.6 90.1) (width 0.4) (layer F.Cu) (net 2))
 (segment (start 139.6 90.1) (end 139.6 92.5) (width 0.4) (layer F.Cu) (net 2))
 (segment (start 135.6 90.1) (end 135.6 87.7) (width 0.4) (layer F.Cu) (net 2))
 (segment (start 135.6 90.1) (end 135.6 92.5) (width 0.4) (layer F.Cu) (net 2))
 (segment (start 131.6 90.1) (end 131.6 87.7) (width 0.4) (layer F.Cu) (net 2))
 (segment (start 135.6 90.1) (end 131.6 90.1) (width 0.4) (layer F.Cu) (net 2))
 (segment (start 131.6 90.1) (end 131.6 92.5) (width 0.4) (layer F.Cu) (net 2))
 (segment (start 127.6 90.1) (end 127.6 92.5) (width 0.4) (layer F.Cu) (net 2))
 (segment (start 131.6 90.1) (end 127.6 90.1) (width 0.4) (layer F.Cu) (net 2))
 (segment (start 127.6 90.1) (end 127.6 87.7) (width 0.4) (layer F.Cu) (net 2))
 (segment (start 171.6 87.7) (end 171.6 92.5) (width 0.4) (layer B.Cu) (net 2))
 (segment (start 122.5 90.1) (end 127.6 90.1) (width 0.4) (layer F.Cu) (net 2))
 (segment (start 118.78 86.38) (end 122.5 90.1) (width 0.4) (layer F.Cu) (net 2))
 (segment (start 122.5 90.1) (end 171.6 90.1) (width 0.4) (layer B.Cu) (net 2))
 (segment (start 118.78 86.38) (end 122.5 90.1) (width 0.4) (layer B.Cu) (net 2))
 (segment (start 167.6 90.1) (end 167.6 87.7) (width 0.4) (layer B.Cu) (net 2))
 (segment (start 167.6 90.1) (end 167.6 92.5) (width 0.4) (layer B.Cu) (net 2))
 (segment (start 163.6 90.1) (end 163.6 87.7) (width 0.4) (layer B.Cu) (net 2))
 (segment (start 163.6 90.1) (end 163.6 92.5) (width 0.4) (layer B.Cu) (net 2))
 (segment (start 159.6 90.1) (end 159.6 87.7) (width 0.4) (layer B.Cu) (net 2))
 (segment (start 159.6 90.1) (end 159.6 92.5) (width 0.4) (layer B.Cu) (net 2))
 (segment (start 155.6 90.1) (end 155.6 87.7) (width 0.4) (layer B.Cu) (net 2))
 (segment (start 155.6 90.1) (end 155.6 92.5) (width 0.4) (layer B.Cu) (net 2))
 (segment (start 151.6 90.1) (end 151.6 87.7) (width 0.4) (layer B.Cu) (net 2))
 (segment (start 151.6 90.1) (end 151.6 92.5) (width 0.4) (layer B.Cu) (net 2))
 (segment (start 147.6 90.1) (end 147.6 87.7) (width 0.4) (layer B.Cu) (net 2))
 (segment (start 147.6 90.1) (end 147.6 92.5) (width 0.4) (layer B.Cu) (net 2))
 (segment (start 143.6 90.1) (end 143.6 87.7) (width 0.4) (layer B.Cu) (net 2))
 (segment (start 143.6 90.1) (end 143.6 92.5) (width 0.4) (layer B.Cu) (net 2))
 (segment (start 139.6 90.1) (end 139.6 87.7) (width 0.4) (layer B.Cu) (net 2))
 (segment (start 139.6 90.1) (end 139.6 92.5) (width 0.4) (layer B.Cu) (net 2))
 (segment (start 135.6 90.1) (end 135.6 87.7) (width 0.4) (layer B.Cu) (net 2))
 (segment (start 135.6 90.1) (end 135.6 92.5) (width 0.4) (layer B.Cu) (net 2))
 (segment (start 131.6 90.1) (end 131.6 87.7) (width 0.4) (layer B.Cu) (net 2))
 (segment (start 131.6 90.1) (end 131.6 92.5) (width 0.4) (layer B.Cu) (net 2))
 (segment (start 127.6 90.1) (end 127.6 87.7) (width 0.4) (layer B.Cu) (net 2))
 (segment (start 127.6 90.1) (end 127.6 92.5) (width 0.4) (layer B.Cu) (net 2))
 (segment (start 118.78 86.38) (end 80.3 86.38) (width 0.4) (layer F.Cu) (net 2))
 (segment (start 118.78 86.38) (end 80.3 86.38) (width 0.4) (layer B.Cu) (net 2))
 (segment (start 173.6 91.1) (end 173.6 89.1) (width 0.4) (layer F.Cu) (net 1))
 (segment (start 169.700001 86.699999) (end 169.6 86.8) (width 0.4) (layer F.Cu) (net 1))
 (segment (start 169.6 86.8) (end 169.6 89.1) (width 0.4) (layer F.Cu) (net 1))
 (segment (start 125.6 86.779998) (end 125.6 89.1) (width 0.4) (layer F.Cu) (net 1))
 (segment (start 125.679999 86.699999) (end 125.6 86.779998) (width 0.4) (layer F.Cu) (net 1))
 (segment (start 170.300001 86.699999) (end 169.700001 86.699999) (width 0.4) (layer F.Cu) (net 1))
 (segment (start 173.199999 86.699999) (end 170.300001 86.699999) (width 0.4) (layer F.Cu) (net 1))
 (segment (start 173.520001 86.699999) (end 173.199999 86.699999) (width 0.4) (layer F.Cu) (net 1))
 (segment (start 173.600001 86.779999) (end 173.520001 86.699999) (width 0.4) (layer F.Cu) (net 1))
 (segment (start 173.6 89.1) (end 173.600001 86.779999) (width 0.4) (layer F.Cu) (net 1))
 (segment (start 173.6 93.3) (end 173.4 93.5) (width 0.4) (layer F.Cu) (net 1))
 (segment (start 173.6 91.1) (end 173.6 93.3) (width 0.4) (layer F.Cu) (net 1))
 (segment (start 169.6 93.5) (end 169.6 91.1) (width 0.4) (layer F.Cu) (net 1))
 (segment (start 173.4 93.5) (end 169.6 93.5) (width 0.4) (layer F.Cu) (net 1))
 (segment (start 165.6 93.5) (end 165.6 91.1) (width 0.4) (layer F.Cu) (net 1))
 (segment (start 169.6 93.5) (end 165.6 93.5) (width 0.4) (layer F.Cu) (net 1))
 (segment (start 165.600001 86.699999) (end 165.6 86.779998) (width 0.4) (layer F.Cu) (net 1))
 (segment (start 165.6 86.779998) (end 165.6 89.1) (width 0.4) (layer F.Cu) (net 1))
 (segment (start 170.300001 86.699999) (end 165.600001 86.699999) (width 0.4) (layer F.Cu) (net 1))
 (segment (start 161.6 86.779998) (end 161.6 89.1) (width 0.4) (layer F.Cu) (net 1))
 (segment (start 161.600001 86.699999) (end 161.6 86.779998) (width 0.4) (layer F.Cu) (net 1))
 (segment (start 165.600001 86.699999) (end 161.600001 86.699999) (width 0.4) (layer F.Cu) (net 1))
 (segment (start 161.6 93.5) (end 161.6 91.1) (width 0.4) (layer F.Cu) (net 1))
 (segment (start 165.6 93.5) (end 161.6 93.5) (width 0.4) (layer F.Cu) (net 1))
 (segment (start 157.6 93.5) (end 157.6 91.1) (width 0.4) (layer F.Cu) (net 1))
 (segment (start 161.6 93.5) (end 157.6 93.5) (width 0.4) (layer F.Cu) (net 1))
 (segment (start 157.600001 86.699999) (end 157.6 86.779998) (width 0.4) (layer F.Cu) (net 1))
 (segment (start 161.600001 86.699999) (end 157.600001 86.699999) (width 0.4) (layer F.Cu) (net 1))
 (segment (start 157.6 86.779998) (end 157.6 89.1) (width 0.4) (layer F.Cu) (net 1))
 (segment (start 153.6 86.779998) (end 153.6 89.1) (width 0.4) (layer F.Cu) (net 1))
 (segment (start 153.600001 86.699999) (end 153.6 86.779998) (width 0.4) (layer F.Cu) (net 1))
 (segment (start 157.600001 86.699999) (end 153.600001 86.699999) (width 0.4) (layer F.Cu) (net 1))
 (segment (start 153.6 93.5) (end 153.6 91.1) (width 0.4) (layer F.Cu) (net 1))
 (segment (start 157.6 93.5) (end 153.6 93.5) (width 0.4) (layer F.Cu) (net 1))
 (segment (start 149.6 86.779998) (end 149.6 89.1) (width 0.4) (layer F.Cu) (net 1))
 (segment (start 149.600001 86.699999) (end 149.6 86.779998) (width 0.4) (layer F.Cu) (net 1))
 (segment (start 153.600001 86.699999) (end 149.600001 86.699999) (width 0.4) (layer F.Cu) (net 1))
 (segment (start 149.6 93.5) (end 149.6 91.1) (width 0.4) (layer F.Cu) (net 1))
 (segment (start 153.6 93.5) (end 149.6 93.5) (width 0.4) (layer F.Cu) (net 1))
 (segment (start 145.6 93.5) (end 145.6 91.1) (width 0.4) (layer F.Cu) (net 1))
 (segment (start 149.6 93.5) (end 145.6 93.5) (width 0.4) (layer F.Cu) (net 1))
 (segment (start 145.6 86.779998) (end 145.6 89.1) (width 0.4) (layer F.Cu) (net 1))
 (segment (start 145.599999 86.699999) (end 145.6 86.779998) (width 0.4) (layer F.Cu) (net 1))
 (segment (start 149.600001 86.699999) (end 145.599999 86.699999) (width 0.4) (layer F.Cu) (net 1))
 (segment (start 141.600001 86.699999) (end 141.6 86.779998) (width 0.4) (layer F.Cu) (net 1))
 (segment (start 141.6 86.779998) (end 141.6 89.1) (width 0.4) (layer F.Cu) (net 1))
 (segment (start 145.599999 86.699999) (end 141.600001 86.699999) (width 0.4) (layer F.Cu) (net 1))
 (segment (start 141.6 93.5) (end 141.6 91.1) (width 0.4) (layer F.Cu) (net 1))
 (segment (start 145.6 93.5) (end 141.6 93.5) (width 0.4) (layer F.Cu) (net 1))
 (segment (start 137.6 93.5) (end 137.6 91.1) (width 0.4) (layer F.Cu) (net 1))
 (segment (start 141.6 93.5) (end 137.6 93.5) (width 0.4) (layer F.Cu) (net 1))
 (segment (start 137.6 86.779998) (end 137.6 89.1) (width 0.4) (layer F.Cu) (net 1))
 (segment (start 137.600001 86.699999) (end 137.6 86.779998) (width 0.4) (layer F.Cu) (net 1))
 (segment (start 141.600001 86.699999) (end 137.600001 86.699999) (width 0.4) (layer F.Cu) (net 1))
 (segment (start 133.6 93.5) (end 133.6 91.1) (width 0.4) (layer F.Cu) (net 1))
 (segment (start 137.6 93.5) (end 133.6 93.5) (width 0.4) (layer F.Cu) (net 1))
 (segment (start 133.6 86.779998) (end 133.6 89.1) (width 0.4) (layer F.Cu) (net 1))
 (segment (start 133.600001 86.699999) (end 133.6 86.779998) (width 0.4) (layer F.Cu) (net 1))
 (segment (start 137.600001 86.699999) (end 133.600001 86.699999) (width 0.4) (layer F.Cu) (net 1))
 (segment (start 129.600001 86.699999) (end 129.6 86.779998) (width 0.4) (layer F.Cu) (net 1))
 (segment (start 129.6 86.779998) (end 129.6 89.1) (width 0.4) (layer F.Cu) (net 1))
 (segment (start 133.600001 86.699999) (end 129.600001 86.699999) (width 0.4) (layer F.Cu) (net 1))
 (segment (start 129.600001 86.699999) (end 125.679999 86.699999) (width 0.4) (layer F.Cu) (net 1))
 (segment (start 129.6 93.5) (end 129.6 91.1) (width 0.4) (layer F.Cu) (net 1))
 (segment (start 133.6 93.5) (end 129.6 93.5) (width 0.4) (layer F.Cu) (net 1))
 (segment (start 125.6 93.5) (end 125.6 91.1) (width 0.4) (layer F.Cu) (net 1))
 (segment (start 129.6 93.5) (end 125.6 93.5) (width 0.4) (layer F.Cu) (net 1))
 (segment (start 173.6 89.1) (end 173.6 91.1) (width 0.4) (layer B.Cu) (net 1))
 (segment (start 173.6 93.3) (end 173.4 93.5) (width 0.4) (layer B.Cu) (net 1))
 (segment (start 173.6 91.1) (end 173.6 93.3) (width 0.4) (layer B.Cu) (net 1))
 (segment (start 125.6 86.779998) (end 125.6 89.1) (width 0.4) (layer B.Cu) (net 1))
 (segment (start 125.679999 86.699999) (end 125.6 86.779998) (width 0.4) (layer B.Cu) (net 1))
 (segment (start 173.6 86.9) (end 173.4 86.7) (width 0.4) (layer B.Cu) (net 1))
 (segment (start 173.6 89.1) (end 173.6 86.9) (width 0.4) (layer B.Cu) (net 1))
 (segment (start 129.6 86.779998) (end 129.6 89.1) (width 0.4) (layer B.Cu) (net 1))
 (segment (start 129.599999 86.699999) (end 129.6 86.779998) (width 0.4) (layer B.Cu) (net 1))
 (segment (start 129.599999 86.699999) (end 125.679999 86.699999) (width 0.4) (layer B.Cu) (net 1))
 (segment (start 133.6 86.7) (end 133.6 89.1) (width 0.4) (layer B.Cu) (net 1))
 (segment (start 133.6 86.7) (end 129.599999 86.699999) (width 0.4) (layer B.Cu) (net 1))
 (segment (start 137.6 86.7) (end 137.6 89.1) (width 0.4) (layer B.Cu) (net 1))
 (segment (start 137.6 86.7) (end 133.6 86.7) (width 0.4) (layer B.Cu) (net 1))
 (segment (start 141.6 86.7) (end 141.6 89.1) (width 0.4) (layer B.Cu) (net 1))
 (segment (start 141.6 86.7) (end 137.6 86.7) (width 0.4) (layer B.Cu) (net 1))
 (segment (start 145.6 86.7) (end 145.6 89.1) (width 0.4) (layer B.Cu) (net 1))
 (segment (start 145.6 86.7) (end 141.6 86.7) (width 0.4) (layer B.Cu) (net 1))
 (segment (start 149.6 86.7) (end 149.6 89.1) (width 0.4) (layer B.Cu) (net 1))
 (segment (start 149.6 86.7) (end 145.6 86.7) (width 0.4) (layer B.Cu) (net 1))
 (segment (start 153.6 86.7) (end 153.6 89.1) (width 0.4) (layer B.Cu) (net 1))
 (segment (start 153.6 86.7) (end 149.6 86.7) (width 0.4) (layer B.Cu) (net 1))
 (segment (start 157.6 86.7) (end 157.6 89.1) (width 0.4) (layer B.Cu) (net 1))
 (segment (start 157.6 86.7) (end 153.6 86.7) (width 0.4) (layer B.Cu) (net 1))
 (segment (start 161.6 86.7) (end 161.6 89.1) (width 0.4) (layer B.Cu) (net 1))
 (segment (start 161.6 86.7) (end 157.6 86.7) (width 0.4) (layer B.Cu) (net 1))
 (segment (start 165.6 86.7) (end 165.6 89.1) (width 0.4) (layer B.Cu) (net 1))
 (segment (start 165.6 86.7) (end 161.6 86.7) (width 0.4) (layer B.Cu) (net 1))
 (segment (start 169.6 86.7) (end 169.6 89.1) (width 0.4) (layer B.Cu) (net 1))
 (segment (start 173.4 86.7) (end 169.6 86.7) (width 0.4) (layer B.Cu) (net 1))
 (segment (start 169.6 86.7) (end 165.6 86.7) (width 0.4) (layer B.Cu) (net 1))
 (segment (start 169.6 93.5) (end 169.6 91.1) (width 0.4) (layer B.Cu) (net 1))
 (segment (start 165.6 93.5) (end 165.6 91.1) (width 0.4) (layer B.Cu) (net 1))
 (segment (start 161.6 93.5) (end 161.6 91.1) (width 0.4) (layer B.Cu) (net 1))
 (segment (start 157.5 93.5) (end 157.6 93.4) (width 0.4) (layer B.Cu) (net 1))
 (segment (start 173.4 93.5) (end 157.5 93.5) (width 0.4) (layer B.Cu) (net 1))
 (segment (start 157.6 93.4) (end 157.6 91.1) (width 0.4) (layer B.Cu) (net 1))
 (segment (start 153.6 93.5) (end 153.6 91.1) (width 0.4) (layer B.Cu) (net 1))
 (segment (start 149.6 93.5) (end 149.6 91.1) (width 0.4) (layer B.Cu) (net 1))
 (segment (start 145.6 93.5) (end 145.6 91.1) (width 0.4) (layer B.Cu) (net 1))
 (segment (start 141.6 93.5) (end 141.6 91.1) (width 0.4) (layer B.Cu) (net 1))
 (segment (start 137.6 93.5) (end 137.6 91.1) (width 0.4) (layer B.Cu) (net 1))
 (segment (start 133.6 93.5) (end 133.6 91.1) (width 0.4) (layer B.Cu) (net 1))
 (segment (start 129.6 93.5) (end 129.6 91.1) (width 0.4) (layer B.Cu) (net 1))
 (segment (start 125.6 93.5) (end 125.6 91.1) (width 0.4) (layer B.Cu) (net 1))
 (segment (start 85.89 93.5) (end 85.1 92.71) (width 0.4) (layer B.Cu) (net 1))
 (segment (start 157.5 93.5) (end 85.89 93.5) (width 0.4) (layer B.Cu) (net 1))
 (segment (start 85.89 93.5) (end 85.1 92.71) (width 0.4) (layer F.Cu) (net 1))
 (segment (start 125.6 93.5) (end 85.89 93.5) (width 0.4) (layer F.Cu) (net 1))
 (segment (start 83.81 94) (end 85.1 92.71) (width 0.4) (layer F.Cu) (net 1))
 (segment (start 80.3 94) (end 83.81 94) (width 0.4) (layer F.Cu) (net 1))
 (segment (start 84.13 87.63) (end 85.1 87.63) (width 0.4) (layer F.Cu) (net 3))
 (segment (start 80.3 91.46) (end 84.13 87.63) (width 0.4) (layer F.Cu) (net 3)))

